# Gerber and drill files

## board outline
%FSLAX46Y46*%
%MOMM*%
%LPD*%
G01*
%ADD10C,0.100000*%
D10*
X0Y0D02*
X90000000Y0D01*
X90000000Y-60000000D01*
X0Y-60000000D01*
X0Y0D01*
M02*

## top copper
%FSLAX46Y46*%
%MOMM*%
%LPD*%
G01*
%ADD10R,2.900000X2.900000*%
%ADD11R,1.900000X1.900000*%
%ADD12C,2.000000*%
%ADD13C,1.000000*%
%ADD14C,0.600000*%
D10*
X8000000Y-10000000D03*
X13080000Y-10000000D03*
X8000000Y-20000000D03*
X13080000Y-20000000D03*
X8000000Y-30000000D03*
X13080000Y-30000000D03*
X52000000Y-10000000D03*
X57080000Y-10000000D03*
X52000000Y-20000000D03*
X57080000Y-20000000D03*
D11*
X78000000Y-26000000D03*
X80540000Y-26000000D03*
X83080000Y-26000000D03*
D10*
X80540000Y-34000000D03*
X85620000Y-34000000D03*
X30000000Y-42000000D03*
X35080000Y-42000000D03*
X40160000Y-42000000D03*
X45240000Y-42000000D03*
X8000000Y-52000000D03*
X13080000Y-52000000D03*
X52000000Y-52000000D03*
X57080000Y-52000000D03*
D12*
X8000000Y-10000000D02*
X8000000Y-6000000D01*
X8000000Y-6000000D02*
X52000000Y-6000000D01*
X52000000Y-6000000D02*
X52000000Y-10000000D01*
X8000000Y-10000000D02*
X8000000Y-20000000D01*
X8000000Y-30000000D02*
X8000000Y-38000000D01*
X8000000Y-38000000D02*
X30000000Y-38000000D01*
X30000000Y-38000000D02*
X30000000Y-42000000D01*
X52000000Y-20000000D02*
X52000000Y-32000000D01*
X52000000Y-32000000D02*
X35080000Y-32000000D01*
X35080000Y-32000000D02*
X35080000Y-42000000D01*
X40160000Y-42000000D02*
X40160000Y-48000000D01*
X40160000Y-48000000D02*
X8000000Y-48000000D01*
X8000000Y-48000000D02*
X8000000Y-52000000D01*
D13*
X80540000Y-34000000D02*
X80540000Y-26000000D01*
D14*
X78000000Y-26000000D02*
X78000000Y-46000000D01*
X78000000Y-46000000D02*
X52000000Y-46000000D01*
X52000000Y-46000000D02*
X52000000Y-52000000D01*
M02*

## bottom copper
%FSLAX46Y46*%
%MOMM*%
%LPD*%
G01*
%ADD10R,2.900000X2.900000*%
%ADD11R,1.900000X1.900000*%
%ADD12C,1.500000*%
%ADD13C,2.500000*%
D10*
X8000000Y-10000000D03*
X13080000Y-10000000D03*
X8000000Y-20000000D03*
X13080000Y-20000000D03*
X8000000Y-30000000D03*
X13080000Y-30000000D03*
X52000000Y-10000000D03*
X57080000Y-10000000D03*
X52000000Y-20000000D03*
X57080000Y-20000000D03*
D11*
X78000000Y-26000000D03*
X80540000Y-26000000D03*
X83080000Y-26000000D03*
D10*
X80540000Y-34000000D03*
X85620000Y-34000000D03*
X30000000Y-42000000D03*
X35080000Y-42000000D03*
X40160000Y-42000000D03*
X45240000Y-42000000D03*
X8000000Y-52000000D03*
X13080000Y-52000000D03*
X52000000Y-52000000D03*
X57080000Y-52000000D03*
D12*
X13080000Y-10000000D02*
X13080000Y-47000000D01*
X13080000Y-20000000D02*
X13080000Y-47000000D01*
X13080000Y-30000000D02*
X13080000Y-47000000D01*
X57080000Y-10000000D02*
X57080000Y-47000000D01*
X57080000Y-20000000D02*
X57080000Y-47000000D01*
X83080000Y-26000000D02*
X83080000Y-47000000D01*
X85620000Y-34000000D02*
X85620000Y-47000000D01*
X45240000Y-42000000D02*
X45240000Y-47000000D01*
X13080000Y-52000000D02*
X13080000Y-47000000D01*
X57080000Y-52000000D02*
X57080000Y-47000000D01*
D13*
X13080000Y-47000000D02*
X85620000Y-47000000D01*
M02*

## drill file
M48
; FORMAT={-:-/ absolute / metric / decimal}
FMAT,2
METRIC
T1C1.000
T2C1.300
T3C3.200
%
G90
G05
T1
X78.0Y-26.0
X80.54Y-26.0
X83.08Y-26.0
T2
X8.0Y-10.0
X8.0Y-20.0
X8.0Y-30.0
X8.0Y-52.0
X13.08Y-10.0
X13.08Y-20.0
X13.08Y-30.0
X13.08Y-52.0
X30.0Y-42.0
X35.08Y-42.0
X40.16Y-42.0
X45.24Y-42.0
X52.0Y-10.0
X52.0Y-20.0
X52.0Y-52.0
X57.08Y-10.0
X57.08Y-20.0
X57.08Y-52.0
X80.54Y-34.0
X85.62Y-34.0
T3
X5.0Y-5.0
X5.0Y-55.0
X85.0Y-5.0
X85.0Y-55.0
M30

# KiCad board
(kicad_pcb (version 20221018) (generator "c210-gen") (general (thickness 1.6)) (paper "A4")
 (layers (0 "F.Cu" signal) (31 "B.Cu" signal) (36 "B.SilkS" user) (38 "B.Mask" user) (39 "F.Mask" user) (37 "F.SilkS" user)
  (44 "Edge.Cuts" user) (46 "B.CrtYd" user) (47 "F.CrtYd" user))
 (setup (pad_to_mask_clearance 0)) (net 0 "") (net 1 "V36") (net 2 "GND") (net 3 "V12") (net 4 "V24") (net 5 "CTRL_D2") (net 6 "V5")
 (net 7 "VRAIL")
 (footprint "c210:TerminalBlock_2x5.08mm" (layer "F.Cu") (at 8 10)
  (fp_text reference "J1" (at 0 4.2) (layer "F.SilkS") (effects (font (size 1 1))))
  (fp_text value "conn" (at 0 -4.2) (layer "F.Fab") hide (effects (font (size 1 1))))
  (pad "1" thru_hole rect (at 0.0 0) (size 2.9 2.9) (drill 1.3) (layers "*.Cu" "*.Mask") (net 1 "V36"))
  (pad "2" thru_hole rect (at 5.08 0) (size 2.9 2.9) (drill 1.3) (layers "*.Cu" "*.Mask") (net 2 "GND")))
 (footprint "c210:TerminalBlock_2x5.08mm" (layer "F.Cu") (at 8 20)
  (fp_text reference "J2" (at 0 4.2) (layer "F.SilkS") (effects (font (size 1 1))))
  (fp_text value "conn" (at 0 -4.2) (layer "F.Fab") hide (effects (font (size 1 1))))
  (pad "1" thru_hole rect (at 0.0 0) (size 2.9 2.9) (drill 1.3) (layers "*.Cu" "*.Mask") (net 1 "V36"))
  (pad "2" thru_hole rect (at 5.08 0) (size 2.9 2.9) (drill 1.3) (layers "*.Cu" "*.Mask") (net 2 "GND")))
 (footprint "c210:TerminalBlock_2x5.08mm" (layer "F.Cu") (at 8 30)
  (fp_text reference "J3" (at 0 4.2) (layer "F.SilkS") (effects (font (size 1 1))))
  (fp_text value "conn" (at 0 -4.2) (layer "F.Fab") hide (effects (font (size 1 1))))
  (pad "1" thru_hole rect (at 0.0 0) (size 2.9 2.9) (drill 1.3) (layers "*.Cu" "*.Mask") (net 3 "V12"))
  (pad "2" thru_hole rect (at 5.08 0) (size 2.9 2.9) (drill 1.3) (layers "*.Cu" "*.Mask") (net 2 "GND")))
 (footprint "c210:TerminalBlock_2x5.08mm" (layer "F.Cu") (at 52 10)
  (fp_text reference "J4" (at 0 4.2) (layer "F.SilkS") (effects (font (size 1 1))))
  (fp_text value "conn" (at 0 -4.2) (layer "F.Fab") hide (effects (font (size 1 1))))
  (pad "1" thru_hole rect (at 0.0 0) (size 2.9 2.9) (drill 1.3) (layers "*.Cu" "*.Mask") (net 1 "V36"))
  (pad "2" thru_hole rect (at 5.08 0) (size 2.9 2.9) (drill 1.3) (layers "*.Cu" "*.Mask") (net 2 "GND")))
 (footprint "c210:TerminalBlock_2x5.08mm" (layer "F.Cu") (at 52 20)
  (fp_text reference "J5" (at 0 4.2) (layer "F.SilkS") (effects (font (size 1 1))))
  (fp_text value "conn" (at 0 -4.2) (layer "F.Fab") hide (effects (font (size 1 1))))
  (pad "1" thru_hole rect (at 0.0 0) (size 2.9 2.9) (drill 1.3) (layers "*.Cu" "*.Mask") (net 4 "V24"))
  (pad "2" thru_hole rect (at 5.08 0) (size 2.9 2.9) (drill 1.3) (layers "*.Cu" "*.Mask") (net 2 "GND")))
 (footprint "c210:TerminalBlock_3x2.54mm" (layer "F.Cu") (at 78 26)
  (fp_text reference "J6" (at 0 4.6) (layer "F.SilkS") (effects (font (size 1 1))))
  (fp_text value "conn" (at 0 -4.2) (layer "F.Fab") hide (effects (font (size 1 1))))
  (pad "1" thru_hole rect (at 0.0 0) (size 1.9 1.9) (drill 1.0) (layers "*.Cu" "*.Mask") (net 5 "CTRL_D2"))
  (pad "2" thru_hole rect (at 2.54 0) (size 1.9 1.9) (drill 1.0) (layers "*.Cu" "*.Mask") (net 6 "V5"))
  (pad "3" thru_hole rect (at 5.08 0) (size 1.9 1.9) (drill 1.0) (layers "*.Cu" "*.Mask") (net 2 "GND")))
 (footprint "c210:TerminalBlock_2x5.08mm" (layer "F.Cu") (at 80.54 34)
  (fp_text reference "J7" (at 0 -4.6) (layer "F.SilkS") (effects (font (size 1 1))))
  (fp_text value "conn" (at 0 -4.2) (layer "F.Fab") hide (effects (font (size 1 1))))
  (pad "1" thru_hole rect (at 0.0 0) (size 2.9 2.9) (drill 1.3) (layers "*.Cu" "*.Mask") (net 6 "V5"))
  (pad "2" thru_hole rect (at 5.08 0) (size 2.9 2.9) (drill 1.3) (layers "*.Cu" "*.Mask") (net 2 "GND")))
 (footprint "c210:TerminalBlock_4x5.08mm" (layer "F.Cu") (at 30 42)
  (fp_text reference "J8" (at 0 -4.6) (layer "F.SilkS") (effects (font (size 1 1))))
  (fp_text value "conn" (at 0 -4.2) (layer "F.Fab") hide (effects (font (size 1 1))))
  (pad "1" thru_hole rect (at 0.0 0) (size 2.9 2.9) (drill 1.3) (layers "*.Cu" "*.Mask") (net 3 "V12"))
  (pad "2" thru_hole rect (at 5.08 0) (size 2.9 2.9) (drill 1.3) (layers "*.Cu" "*.Mask") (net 4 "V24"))
  (pad "3" thru_hole rect (at 10.16 0) (size 2.9 2.9) (drill 1.3) (layers "*.Cu" "*.Mask") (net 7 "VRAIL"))
  (pad "4" thru_hole rect (at 15.24 0) (size 2.9 2.9) (drill 1.3) (layers "*.Cu" "*.Mask") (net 2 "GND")))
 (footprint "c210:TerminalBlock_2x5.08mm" (layer "F.Cu") (at 8 52)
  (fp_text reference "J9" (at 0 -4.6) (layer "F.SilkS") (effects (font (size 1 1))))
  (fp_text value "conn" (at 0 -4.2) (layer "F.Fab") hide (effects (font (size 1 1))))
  (pad "1" thru_hole rect (at 0.0 0) (size 2.9 2.9) (drill 1.3) (layers "*.Cu" "*.Mask") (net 7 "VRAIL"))
  (pad "2" thru_hole rect (at 5.08 0) (size 2.9 2.9) (drill 1.3) (layers "*.Cu" "*.Mask") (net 2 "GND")))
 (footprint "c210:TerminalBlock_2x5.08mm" (layer "F.Cu") (at 52 52)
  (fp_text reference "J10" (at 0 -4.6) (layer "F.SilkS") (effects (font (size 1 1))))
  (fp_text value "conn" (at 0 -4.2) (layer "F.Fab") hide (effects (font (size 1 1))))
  (pad "1" thru_hole rect (at 0.0 0) (size 2.9 2.9) (drill 1.3) (layers "*.Cu" "*.Mask") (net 5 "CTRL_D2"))
  (pad "2" thru_hole rect (at 5.08 0) (size 2.9 2.9) (drill 1.3) (layers "*.Cu" "*.Mask") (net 2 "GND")))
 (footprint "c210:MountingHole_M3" (layer "F.Cu") (at 5 5)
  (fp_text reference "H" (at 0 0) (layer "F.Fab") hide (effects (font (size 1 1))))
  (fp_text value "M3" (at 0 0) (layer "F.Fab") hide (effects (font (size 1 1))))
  (pad "" np_thru_hole circle (at 0 0) (size 3.2 3.2) (drill 3.2) (layers "F.Mask" "B.Mask")))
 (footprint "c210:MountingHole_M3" (layer "F.Cu") (at 85 5)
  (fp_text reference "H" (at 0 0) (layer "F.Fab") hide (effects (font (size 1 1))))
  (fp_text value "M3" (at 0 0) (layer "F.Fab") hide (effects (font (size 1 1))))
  (pad "" np_thru_hole circle (at 0 0) (size 3.2 3.2) (drill 3.2) (layers "F.Mask" "B.Mask")))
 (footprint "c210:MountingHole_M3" (layer "F.Cu") (at 5 55)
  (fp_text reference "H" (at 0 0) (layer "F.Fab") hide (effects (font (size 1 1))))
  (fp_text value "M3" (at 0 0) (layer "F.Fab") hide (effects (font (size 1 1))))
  (pad "" np_thru_hole circle (at 0 0) (size 3.2 3.2) (drill 3.2) (layers "F.Mask" "B.Mask")))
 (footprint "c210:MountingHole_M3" (layer "F.Cu") (at 85 55)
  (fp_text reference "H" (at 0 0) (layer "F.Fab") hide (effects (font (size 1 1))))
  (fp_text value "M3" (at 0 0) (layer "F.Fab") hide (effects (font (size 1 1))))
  (pad "" np_thru_hole circle (at 0 0) (size 3.2 3.2) (drill 3.2) (layers "F.Mask" "B.Mask")))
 (segment (start 8.0 10) (end 8 6) (width 2.0) (layer "F.Cu") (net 1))
 (segment (start 8 6) (end 52 6) (width 2.0) (layer "F.Cu") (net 1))
 (segment (start 52 6) (end 52.0 10) (width 2.0) (layer "F.Cu") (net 1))
 (segment (start 8.0 10) (end 8.0 20) (width 2.0) (layer "F.Cu") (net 1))
 (segment (start 8.0 30) (end 8 38) (width 2.0) (layer "F.Cu") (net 3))
 (segment (start 8 38) (end 30 38) (width 2.0) (layer "F.Cu") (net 3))
 (segment (start 30 38) (end 30.0 42) (width 2.0) (layer "F.Cu") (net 3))
 (segment (start 52.0 20) (end 52 32) (width 2.0) (layer "F.Cu") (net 4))
 (segment (start 52 32) (end 35.08 32) (width 2.0) (layer "F.Cu") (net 4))
 (segment (start 35.08 32) (end 35.08 42) (width 2.0) (layer "F.Cu") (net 4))
 (segment (start 40.16 42) (end 40.16 48) (width 2.0) (layer "F.Cu") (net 7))
 (segment (start 40.16 48) (end 8 48) (width 2.0) (layer "F.Cu") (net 7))
 (segment (start 8 48) (end 8.0 52) (width 2.0) (layer "F.Cu") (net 7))
 (segment (start 80.54 34) (end 80.54 26) (width 1.0) (layer "F.Cu") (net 6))
 (segment (start 78.0 26) (end 78 46) (width 0.6) (layer "F.Cu") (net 5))
 (segment (start 78 46) (end 52 46) (width 0.6) (layer "F.Cu") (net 5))
 (segment (start 52 46) (end 52.0 52) (width 0.6) (layer "F.Cu") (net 5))
 (segment (start 13.08 10) (end 13.08 47) (width 1.5) (layer "B.Cu") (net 2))
 (segment (start 13.08 20) (end 13.08 47) (width 1.5) (layer "B.Cu") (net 2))
 (segment (start 13.08 30) (end 13.08 47) (width 1.5) (layer "B.Cu") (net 2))
 (segment (start 57.08 10) (end 57.08 47) (width 1.5) (layer "B.Cu") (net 2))
 (segment (start 57.08 20) (end 57.08 47) (width 1.5) (layer "B.Cu") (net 2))
 (segment (start 83.08 26) (end 83.08 47) (width 1.5) (layer "B.Cu") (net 2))
 (segment (start 85.62 34) (end 85.62 47) (width 1.5) (layer "B.Cu") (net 2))
 (segment (start 45.24 42) (end 45.24 47) (width 1.5) (layer "B.Cu") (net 2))
 (segment (start 13.08 52) (end 13.08 47) (width 1.5) (layer "B.Cu") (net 2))
 (segment (start 57.08 52) (end 57.08 47) (width 1.5) (layer "B.Cu") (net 2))
 (segment (start 13.08 47) (end 85.62 47) (width 2.5) (layer "B.Cu") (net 2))
 (gr_rect (start 0 0) (end 90 60) (stroke (width 0.1) (type default)) (fill none) (layer "Edge.Cuts")))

